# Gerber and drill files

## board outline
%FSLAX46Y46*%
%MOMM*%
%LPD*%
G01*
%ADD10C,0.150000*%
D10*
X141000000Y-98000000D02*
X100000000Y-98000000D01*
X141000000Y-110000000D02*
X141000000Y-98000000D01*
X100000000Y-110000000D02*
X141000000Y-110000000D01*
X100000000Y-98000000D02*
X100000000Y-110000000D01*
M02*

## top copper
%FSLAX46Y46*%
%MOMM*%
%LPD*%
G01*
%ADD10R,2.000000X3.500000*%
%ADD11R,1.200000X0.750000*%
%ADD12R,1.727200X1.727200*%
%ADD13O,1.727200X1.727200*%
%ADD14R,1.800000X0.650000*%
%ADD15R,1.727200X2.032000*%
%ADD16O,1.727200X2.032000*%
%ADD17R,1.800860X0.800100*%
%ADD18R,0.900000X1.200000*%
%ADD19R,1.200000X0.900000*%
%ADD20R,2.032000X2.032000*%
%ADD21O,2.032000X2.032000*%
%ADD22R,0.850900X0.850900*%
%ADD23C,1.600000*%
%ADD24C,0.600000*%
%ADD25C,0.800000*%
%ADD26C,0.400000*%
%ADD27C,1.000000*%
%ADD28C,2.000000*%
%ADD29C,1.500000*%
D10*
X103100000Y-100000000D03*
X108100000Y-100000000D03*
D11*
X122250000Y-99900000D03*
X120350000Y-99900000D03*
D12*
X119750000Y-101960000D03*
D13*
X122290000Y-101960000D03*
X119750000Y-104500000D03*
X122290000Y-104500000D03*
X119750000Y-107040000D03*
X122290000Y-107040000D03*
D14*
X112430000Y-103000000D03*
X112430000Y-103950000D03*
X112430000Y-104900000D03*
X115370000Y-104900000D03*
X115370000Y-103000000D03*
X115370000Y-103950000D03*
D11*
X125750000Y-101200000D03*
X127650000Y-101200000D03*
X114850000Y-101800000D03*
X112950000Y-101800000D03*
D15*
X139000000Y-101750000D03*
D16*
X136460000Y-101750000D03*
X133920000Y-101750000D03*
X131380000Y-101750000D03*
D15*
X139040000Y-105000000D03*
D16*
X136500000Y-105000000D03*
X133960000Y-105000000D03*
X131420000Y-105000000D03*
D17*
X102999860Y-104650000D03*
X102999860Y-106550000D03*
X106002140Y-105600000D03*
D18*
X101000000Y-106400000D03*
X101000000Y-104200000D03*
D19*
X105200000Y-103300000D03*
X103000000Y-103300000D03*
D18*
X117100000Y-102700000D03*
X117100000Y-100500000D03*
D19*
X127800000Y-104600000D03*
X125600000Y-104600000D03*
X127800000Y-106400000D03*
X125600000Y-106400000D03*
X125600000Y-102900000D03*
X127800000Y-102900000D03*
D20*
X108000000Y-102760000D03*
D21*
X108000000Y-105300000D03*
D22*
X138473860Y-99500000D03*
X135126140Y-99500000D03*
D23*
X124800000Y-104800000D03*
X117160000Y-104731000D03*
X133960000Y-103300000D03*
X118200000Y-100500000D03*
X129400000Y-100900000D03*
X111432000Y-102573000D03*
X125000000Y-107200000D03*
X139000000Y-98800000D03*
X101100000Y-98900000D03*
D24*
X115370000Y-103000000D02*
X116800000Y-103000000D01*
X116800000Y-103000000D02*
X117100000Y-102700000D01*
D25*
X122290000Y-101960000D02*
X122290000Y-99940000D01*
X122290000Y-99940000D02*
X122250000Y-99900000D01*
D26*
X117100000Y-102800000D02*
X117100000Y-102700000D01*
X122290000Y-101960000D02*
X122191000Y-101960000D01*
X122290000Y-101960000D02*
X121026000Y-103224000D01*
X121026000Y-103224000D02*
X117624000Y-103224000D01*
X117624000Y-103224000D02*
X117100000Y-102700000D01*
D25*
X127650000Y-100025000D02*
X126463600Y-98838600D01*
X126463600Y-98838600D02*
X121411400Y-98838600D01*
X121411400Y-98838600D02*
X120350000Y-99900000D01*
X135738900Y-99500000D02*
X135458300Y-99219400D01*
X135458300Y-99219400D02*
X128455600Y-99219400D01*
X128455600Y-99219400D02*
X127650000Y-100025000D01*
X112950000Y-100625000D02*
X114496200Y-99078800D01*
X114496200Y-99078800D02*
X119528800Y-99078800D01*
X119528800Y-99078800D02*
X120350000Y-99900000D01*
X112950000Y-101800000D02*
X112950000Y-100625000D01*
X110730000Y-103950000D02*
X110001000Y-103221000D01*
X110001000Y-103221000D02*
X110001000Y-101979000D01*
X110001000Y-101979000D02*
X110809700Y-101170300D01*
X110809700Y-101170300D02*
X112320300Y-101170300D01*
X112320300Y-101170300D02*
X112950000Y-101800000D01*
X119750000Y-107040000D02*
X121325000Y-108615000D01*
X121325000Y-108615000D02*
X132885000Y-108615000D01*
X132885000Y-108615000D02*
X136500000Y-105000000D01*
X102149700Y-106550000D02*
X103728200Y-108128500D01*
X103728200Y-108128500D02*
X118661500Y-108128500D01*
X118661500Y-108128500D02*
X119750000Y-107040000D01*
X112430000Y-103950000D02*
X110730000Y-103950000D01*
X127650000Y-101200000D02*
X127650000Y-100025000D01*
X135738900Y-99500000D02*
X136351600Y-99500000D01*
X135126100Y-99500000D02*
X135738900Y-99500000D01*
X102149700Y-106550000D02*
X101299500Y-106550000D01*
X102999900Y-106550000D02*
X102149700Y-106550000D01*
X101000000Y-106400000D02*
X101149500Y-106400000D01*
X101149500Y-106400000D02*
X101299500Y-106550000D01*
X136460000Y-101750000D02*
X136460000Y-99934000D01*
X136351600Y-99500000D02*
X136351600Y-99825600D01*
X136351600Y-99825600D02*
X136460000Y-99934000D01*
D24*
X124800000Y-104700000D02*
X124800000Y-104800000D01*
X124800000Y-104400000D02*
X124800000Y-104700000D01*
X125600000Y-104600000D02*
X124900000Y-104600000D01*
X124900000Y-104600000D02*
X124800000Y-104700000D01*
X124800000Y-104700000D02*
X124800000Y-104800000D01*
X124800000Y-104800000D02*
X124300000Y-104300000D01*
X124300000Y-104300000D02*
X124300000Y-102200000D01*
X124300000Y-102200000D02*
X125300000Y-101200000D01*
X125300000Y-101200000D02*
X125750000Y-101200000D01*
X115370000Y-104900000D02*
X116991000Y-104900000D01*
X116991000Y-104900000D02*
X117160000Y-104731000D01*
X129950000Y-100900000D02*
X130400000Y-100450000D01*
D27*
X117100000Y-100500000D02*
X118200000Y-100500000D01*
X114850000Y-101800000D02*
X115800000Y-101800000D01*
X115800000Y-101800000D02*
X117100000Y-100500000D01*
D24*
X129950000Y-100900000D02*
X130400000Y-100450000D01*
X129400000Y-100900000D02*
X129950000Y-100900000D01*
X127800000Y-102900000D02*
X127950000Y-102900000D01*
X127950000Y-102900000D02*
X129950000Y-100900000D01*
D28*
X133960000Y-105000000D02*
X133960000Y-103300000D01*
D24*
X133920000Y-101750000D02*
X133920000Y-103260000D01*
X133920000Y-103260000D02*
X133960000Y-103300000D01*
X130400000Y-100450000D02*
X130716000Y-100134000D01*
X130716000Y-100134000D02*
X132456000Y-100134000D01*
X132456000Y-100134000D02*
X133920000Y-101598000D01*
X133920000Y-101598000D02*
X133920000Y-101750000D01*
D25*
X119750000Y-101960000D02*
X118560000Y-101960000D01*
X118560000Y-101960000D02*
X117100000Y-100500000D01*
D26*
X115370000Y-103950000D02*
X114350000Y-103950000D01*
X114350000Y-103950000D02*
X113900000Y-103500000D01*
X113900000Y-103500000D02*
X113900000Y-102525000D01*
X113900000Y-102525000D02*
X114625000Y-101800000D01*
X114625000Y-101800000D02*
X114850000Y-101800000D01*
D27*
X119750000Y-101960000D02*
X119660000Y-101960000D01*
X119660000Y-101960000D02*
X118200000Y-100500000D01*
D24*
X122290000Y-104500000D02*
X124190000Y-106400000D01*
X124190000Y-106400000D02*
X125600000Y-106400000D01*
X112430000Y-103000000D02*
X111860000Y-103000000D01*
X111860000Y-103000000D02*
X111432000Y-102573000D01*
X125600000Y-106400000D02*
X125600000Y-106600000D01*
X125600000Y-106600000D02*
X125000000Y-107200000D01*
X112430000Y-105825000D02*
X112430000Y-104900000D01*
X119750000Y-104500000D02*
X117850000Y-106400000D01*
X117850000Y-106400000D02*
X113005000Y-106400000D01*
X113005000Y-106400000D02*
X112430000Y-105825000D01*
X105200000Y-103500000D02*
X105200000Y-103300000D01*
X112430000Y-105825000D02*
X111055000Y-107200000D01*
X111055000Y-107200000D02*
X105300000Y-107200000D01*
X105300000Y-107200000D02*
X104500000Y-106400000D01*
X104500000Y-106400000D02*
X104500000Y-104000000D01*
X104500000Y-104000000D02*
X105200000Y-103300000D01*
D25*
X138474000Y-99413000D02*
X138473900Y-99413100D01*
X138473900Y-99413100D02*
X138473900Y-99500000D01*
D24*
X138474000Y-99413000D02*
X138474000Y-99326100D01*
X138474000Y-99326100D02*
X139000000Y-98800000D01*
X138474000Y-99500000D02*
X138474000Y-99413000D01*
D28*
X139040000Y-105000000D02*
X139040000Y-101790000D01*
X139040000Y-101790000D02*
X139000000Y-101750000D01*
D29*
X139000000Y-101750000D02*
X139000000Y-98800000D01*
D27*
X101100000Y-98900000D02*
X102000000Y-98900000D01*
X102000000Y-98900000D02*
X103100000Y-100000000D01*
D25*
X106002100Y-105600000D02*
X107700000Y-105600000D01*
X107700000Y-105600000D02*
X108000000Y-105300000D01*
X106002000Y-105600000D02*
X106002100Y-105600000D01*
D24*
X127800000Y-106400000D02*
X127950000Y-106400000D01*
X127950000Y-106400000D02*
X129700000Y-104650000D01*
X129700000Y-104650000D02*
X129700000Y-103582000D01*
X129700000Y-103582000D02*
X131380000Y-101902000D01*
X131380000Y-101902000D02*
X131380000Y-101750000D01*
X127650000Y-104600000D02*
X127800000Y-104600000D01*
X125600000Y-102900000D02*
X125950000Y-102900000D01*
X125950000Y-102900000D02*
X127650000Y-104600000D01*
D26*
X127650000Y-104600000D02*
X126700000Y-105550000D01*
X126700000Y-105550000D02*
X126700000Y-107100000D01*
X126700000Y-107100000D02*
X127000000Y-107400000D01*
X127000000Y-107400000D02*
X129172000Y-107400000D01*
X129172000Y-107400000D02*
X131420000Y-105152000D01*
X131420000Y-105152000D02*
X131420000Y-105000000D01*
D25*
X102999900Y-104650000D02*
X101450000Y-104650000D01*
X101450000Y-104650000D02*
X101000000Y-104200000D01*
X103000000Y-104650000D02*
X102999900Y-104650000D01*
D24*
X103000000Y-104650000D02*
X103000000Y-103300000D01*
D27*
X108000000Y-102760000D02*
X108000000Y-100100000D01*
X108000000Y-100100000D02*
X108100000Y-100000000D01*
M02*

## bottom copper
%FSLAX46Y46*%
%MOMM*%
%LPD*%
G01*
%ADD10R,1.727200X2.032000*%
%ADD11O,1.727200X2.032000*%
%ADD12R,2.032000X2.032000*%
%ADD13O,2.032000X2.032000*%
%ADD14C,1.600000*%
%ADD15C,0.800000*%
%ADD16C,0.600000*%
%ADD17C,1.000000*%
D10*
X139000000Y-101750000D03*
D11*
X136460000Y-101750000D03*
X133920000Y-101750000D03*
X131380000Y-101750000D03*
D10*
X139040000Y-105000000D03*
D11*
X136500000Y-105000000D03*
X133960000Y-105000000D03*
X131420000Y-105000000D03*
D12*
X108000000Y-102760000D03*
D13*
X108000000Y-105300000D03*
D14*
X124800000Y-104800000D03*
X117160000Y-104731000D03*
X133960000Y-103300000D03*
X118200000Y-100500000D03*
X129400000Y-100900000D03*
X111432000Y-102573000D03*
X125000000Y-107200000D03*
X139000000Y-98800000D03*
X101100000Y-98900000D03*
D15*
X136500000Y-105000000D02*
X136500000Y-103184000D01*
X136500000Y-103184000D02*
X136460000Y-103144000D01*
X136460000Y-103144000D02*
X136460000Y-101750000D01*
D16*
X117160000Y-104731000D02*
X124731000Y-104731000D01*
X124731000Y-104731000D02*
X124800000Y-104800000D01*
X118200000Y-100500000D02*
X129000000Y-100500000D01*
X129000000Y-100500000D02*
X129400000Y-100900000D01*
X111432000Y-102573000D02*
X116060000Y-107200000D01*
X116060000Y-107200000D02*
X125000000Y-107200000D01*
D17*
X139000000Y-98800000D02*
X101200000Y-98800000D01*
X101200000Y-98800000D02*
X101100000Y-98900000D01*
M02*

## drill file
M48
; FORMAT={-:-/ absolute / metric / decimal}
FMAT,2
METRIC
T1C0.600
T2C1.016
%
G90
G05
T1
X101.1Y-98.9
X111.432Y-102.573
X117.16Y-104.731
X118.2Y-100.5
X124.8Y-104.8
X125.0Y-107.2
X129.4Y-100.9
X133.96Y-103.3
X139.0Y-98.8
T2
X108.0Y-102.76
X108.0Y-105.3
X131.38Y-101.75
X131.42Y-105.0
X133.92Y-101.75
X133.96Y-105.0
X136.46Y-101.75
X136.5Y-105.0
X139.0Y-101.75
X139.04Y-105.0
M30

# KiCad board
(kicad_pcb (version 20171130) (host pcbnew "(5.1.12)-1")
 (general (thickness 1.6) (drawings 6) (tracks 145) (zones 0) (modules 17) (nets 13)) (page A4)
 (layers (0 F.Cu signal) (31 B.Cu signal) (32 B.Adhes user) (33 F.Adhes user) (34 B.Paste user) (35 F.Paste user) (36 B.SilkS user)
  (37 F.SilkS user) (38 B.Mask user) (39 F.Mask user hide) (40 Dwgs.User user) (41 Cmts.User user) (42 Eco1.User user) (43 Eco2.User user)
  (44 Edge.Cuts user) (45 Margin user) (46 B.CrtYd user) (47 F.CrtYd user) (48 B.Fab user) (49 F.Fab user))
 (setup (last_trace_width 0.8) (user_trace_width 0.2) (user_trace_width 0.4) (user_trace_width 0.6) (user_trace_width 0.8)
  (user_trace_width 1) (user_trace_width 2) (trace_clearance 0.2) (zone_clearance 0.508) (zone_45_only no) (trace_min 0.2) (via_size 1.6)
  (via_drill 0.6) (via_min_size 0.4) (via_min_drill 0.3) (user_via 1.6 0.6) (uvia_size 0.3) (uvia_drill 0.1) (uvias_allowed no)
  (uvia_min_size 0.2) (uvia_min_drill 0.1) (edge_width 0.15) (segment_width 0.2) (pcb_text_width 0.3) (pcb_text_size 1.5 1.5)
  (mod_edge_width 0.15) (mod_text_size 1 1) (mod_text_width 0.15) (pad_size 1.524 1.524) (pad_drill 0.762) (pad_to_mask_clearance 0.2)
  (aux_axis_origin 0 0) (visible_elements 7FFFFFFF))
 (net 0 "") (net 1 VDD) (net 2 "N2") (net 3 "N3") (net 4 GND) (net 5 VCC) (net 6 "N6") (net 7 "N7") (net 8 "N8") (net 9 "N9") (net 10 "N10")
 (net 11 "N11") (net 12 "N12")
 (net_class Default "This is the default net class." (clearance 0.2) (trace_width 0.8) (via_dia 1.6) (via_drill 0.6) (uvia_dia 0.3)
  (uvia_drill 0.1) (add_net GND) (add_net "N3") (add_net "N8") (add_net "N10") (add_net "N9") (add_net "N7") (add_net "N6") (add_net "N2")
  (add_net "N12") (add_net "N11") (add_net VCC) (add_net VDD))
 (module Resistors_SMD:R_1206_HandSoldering (layer F.Cu) (at 105.6 100)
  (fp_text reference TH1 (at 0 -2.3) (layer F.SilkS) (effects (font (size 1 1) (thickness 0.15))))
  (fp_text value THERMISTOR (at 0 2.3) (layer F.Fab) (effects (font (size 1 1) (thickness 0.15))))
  (pad 1 smd rect (at -2.5 0) (size 2 3.5) (layers F.Cu F.Paste F.Mask) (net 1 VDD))
  (pad 2 smd rect (at 2.5 0) (size 2 3.5) (layers F.Cu F.Paste F.Mask) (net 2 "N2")))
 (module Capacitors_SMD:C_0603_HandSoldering (layer F.Cu) (at 121.3 99.9 180)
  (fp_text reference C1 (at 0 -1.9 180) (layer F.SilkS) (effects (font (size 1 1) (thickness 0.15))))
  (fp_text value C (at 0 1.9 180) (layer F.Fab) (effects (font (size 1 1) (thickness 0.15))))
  (pad 1 smd rect (at -0.95 0 180) (size 1.2 0.75) (layers F.Cu F.Paste F.Mask) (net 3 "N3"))
  (pad 2 smd rect (at 0.95 0 180) (size 1.2 0.75) (layers F.Cu F.Paste F.Mask) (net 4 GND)))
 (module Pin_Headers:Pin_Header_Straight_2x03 (layer F.Cu) (at 119.75 101.96)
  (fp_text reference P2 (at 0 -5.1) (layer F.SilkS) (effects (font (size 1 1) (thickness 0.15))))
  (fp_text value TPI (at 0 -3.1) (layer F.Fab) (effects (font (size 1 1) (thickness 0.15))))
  (pad 1 smd rect (at 0 0) (size 1.7272 1.7272) (layers F.Cu F.Paste F.Mask) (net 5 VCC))
  (pad 2 smd oval (at 2.54 0) (size 1.7272 1.7272) (layers F.Cu F.Paste F.Mask) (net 3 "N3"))
  (pad 3 smd oval (at 0 2.54) (size 1.7272 1.7272) (layers F.Cu F.Paste F.Mask) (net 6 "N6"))
  (pad 4 smd oval (at 2.54 2.54) (size 1.7272 1.7272) (layers F.Cu F.Paste F.Mask) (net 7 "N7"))
  (pad 5 smd oval (at 0 5.08) (size 1.7272 1.7272) (layers F.Cu F.Paste F.Mask) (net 4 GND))
  (pad 6 smd oval (at 2.54 5.08) (size 1.7272 1.7272) (layers F.Cu F.Paste F.Mask)))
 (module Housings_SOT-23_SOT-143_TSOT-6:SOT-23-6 (layer F.Cu) (at 113.9 103.95)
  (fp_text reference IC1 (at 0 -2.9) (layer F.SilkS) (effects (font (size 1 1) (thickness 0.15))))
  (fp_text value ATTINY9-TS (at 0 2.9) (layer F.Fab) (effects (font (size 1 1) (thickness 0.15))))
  (pad 1 smd rect (at -1.47 -0.95) (size 1.8 0.65) (layers F.Cu F.Paste F.Mask) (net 7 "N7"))
  (pad 2 smd rect (at -1.47 0) (size 1.8 0.65) (layers F.Cu F.Paste F.Mask) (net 4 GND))
  (pad 3 smd rect (at -1.47 0.95) (size 1.8 0.65) (layers F.Cu F.Paste F.Mask) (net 6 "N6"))
  (pad 4 smd rect (at 1.47 0.95) (size 1.8 0.65) (layers F.Cu F.Paste F.Mask) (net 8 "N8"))
  (pad 6 smd rect (at 1.47 -0.95) (size 1.8 0.65) (layers F.Cu F.Paste F.Mask) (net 3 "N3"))
  (pad 5 smd rect (at 1.47 0) (size 1.8 0.65) (layers F.Cu F.Paste F.Mask) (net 5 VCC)))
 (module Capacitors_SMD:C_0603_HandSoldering (layer F.Cu) (at 126.7 101.2)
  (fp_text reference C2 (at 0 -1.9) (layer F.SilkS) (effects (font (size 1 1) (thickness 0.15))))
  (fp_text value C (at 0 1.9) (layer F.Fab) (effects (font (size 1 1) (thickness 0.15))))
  (pad 1 smd rect (at -0.95 0) (size 1.2 0.75) (layers F.Cu F.Paste F.Mask) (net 8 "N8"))
  (pad 2 smd rect (at 0.95 0) (size 1.2 0.75) (layers F.Cu F.Paste F.Mask) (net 4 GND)))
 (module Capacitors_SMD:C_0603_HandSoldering (layer F.Cu) (at 113.9 101.8 180)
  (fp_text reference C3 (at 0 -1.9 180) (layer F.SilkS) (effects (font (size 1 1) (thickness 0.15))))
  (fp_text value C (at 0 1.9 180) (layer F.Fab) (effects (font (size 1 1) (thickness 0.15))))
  (pad 1 smd rect (at -0.95 0 180) (size 1.2 0.75) (layers F.Cu F.Paste F.Mask) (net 5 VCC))
  (pad 2 smd rect (at 0.95 0 180) (size 1.2 0.75) (layers F.Cu F.Paste F.Mask) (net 4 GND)))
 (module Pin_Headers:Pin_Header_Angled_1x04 (layer B.Cu) (at 139 101.75 90)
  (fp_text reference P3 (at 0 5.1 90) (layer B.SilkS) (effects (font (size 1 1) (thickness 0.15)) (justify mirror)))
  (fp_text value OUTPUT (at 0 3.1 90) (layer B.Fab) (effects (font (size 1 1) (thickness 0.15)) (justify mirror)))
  (pad 1 thru_hole rect (at 0 0 90) (size 2.032 1.7272) (drill 1.016) (layers *.Cu *.Mask B.SilkS) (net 1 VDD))
  (pad 2 thru_hole oval (at 0 -2.54 90) (size 2.032 1.7272) (drill 1.016) (layers *.Cu *.Mask B.SilkS) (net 4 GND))
  (pad 3 thru_hole oval (at 0 -5.08 90) (size 2.032 1.7272) (drill 1.016) (layers *.Cu *.Mask B.SilkS) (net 5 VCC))
  (pad 4 thru_hole oval (at 0 -7.62 90) (size 2.032 1.7272) (drill 1.016) (layers *.Cu *.Mask B.SilkS) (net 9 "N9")))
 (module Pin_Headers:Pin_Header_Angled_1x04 (layer F.Cu) (at 139.04 105 270)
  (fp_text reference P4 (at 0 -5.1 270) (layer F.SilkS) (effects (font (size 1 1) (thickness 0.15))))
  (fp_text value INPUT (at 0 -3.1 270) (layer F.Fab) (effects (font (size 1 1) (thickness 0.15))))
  (pad 1 thru_hole rect (at 0 0 270) (size 2.032 1.7272) (drill 1.016) (layers *.Cu *.Mask F.SilkS) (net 1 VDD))
  (pad 2 thru_hole oval (at 0 2.54 270) (size 2.032 1.7272) (drill 1.016) (layers *.Cu *.Mask F.SilkS) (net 4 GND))
  (pad 3 thru_hole oval (at 0 5.08 270) (size 2.032 1.7272) (drill 1.016) (layers *.Cu *.Mask F.SilkS) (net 5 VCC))
  (pad 4 thru_hole oval (at 0 7.62 270) (size 2.032 1.7272) (drill 1.016) (layers *.Cu *.Mask F.SilkS) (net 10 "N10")))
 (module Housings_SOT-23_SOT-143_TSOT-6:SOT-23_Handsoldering (layer F.Cu) (at 104.501 105.6 270)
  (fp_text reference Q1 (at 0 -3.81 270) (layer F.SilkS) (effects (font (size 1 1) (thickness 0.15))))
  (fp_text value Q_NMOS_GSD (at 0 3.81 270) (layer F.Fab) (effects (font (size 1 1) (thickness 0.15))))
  (pad 1 smd rect (at -0.95 1.50114 270) (size 0.8001 1.80086) (layers F.Cu F.Paste F.Mask) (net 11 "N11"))
  (pad 2 smd rect (at 0.95 1.50114 270) (size 0.8001 1.80086) (layers F.Cu F.Paste F.Mask) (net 4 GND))
  (pad 3 smd rect (at 0 -1.50114 270) (size 0.8001 1.80086) (layers F.Cu F.Paste F.Mask) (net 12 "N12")))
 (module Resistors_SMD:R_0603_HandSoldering (layer F.Cu) (at 101 105.3 90)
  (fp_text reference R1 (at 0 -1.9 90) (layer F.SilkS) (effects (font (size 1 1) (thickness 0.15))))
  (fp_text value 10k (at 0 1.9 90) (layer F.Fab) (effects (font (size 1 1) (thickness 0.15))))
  (pad 1 smd rect (at -1.1 0 90) (size 1.2 0.9) (layers F.Cu F.Paste F.Mask) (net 4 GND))
  (pad 2 smd rect (at 1.1 0 90) (size 1.2 0.9) (layers F.Cu F.Paste F.Mask) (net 11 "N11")))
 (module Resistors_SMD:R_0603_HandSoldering (layer F.Cu) (at 104.1 103.3 180)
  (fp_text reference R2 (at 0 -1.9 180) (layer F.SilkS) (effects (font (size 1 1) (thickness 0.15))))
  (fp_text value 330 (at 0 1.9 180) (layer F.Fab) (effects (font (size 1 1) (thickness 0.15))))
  (pad 1 smd rect (at -1.1 0 180) (size 1.2 0.9) (layers F.Cu F.Paste F.Mask) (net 6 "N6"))
  (pad 2 smd rect (at 1.1 0 180) (size 1.2 0.9) (layers F.Cu F.Paste F.Mask) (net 11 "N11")))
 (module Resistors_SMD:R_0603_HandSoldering (layer F.Cu) (at 117.1 101.6 90)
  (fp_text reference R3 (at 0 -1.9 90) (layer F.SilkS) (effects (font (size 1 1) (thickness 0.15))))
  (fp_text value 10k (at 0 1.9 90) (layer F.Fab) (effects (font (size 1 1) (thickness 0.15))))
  (pad 1 smd rect (at -1.1 0 90) (size 1.2 0.9) (layers F.Cu F.Paste F.Mask) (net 3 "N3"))
  (pad 2 smd rect (at 1.1 0 90) (size 1.2 0.9) (layers F.Cu F.Paste F.Mask) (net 5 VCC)))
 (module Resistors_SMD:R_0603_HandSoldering (layer F.Cu) (at 126.7 104.6 180)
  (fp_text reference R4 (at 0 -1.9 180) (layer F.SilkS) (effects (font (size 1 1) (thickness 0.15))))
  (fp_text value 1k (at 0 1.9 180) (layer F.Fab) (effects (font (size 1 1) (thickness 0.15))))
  (pad 1 smd rect (at -1.1 0 180) (size 1.2 0.9) (layers F.Cu F.Paste F.Mask) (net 10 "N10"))
  (pad 2 smd rect (at 1.1 0 180) (size 1.2 0.9) (layers F.Cu F.Paste F.Mask) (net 8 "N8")))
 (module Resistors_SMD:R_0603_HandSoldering (layer F.Cu) (at 126.7 106.4 180)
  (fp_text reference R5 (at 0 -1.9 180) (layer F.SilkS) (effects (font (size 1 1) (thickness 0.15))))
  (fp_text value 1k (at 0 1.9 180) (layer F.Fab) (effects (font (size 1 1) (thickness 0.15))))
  (pad 1 smd rect (at -1.1 0 180) (size 1.2 0.9) (layers F.Cu F.Paste F.Mask) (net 9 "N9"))
  (pad 2 smd rect (at 1.1 0 180) (size 1.2 0.9) (layers F.Cu F.Paste F.Mask) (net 7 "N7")))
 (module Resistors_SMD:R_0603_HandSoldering (layer F.Cu) (at 126.7 102.9)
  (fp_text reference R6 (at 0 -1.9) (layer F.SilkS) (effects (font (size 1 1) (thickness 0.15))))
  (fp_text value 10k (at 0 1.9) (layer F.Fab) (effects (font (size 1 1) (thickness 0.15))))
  (pad 1 smd rect (at -1.1 0) (size 1.2 0.9) (layers F.Cu F.Paste F.Mask) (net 10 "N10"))
  (pad 2 smd rect (at 1.1 0) (size 1.2 0.9) (layers F.Cu F.Paste F.Mask) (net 5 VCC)))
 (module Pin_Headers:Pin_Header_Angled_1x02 (layer B.Cu) (at 108 102.76 180)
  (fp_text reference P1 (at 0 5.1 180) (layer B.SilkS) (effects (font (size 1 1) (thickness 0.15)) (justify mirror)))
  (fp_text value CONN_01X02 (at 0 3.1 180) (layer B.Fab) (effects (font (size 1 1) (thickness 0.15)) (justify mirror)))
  (pad 1 thru_hole rect (at 0 0 180) (size 2.032 2.032) (drill 1.016) (layers *.Cu *.Mask B.SilkS) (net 2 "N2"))
  (pad 2 thru_hole oval (at 0 -2.54 180) (size 2.032 2.032) (drill 1.016) (layers *.Cu *.Mask B.SilkS) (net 12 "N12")))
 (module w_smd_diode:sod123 (layer F.Cu) (at 136.8 99.5)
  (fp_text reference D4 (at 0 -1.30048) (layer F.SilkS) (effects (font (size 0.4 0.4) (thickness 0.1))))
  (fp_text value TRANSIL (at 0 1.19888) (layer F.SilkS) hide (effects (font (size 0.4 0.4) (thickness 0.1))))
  (pad 2 smd rect (at 1.67386 0) (size 0.8509 0.8509) (layers F.Cu F.Paste F.Mask) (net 1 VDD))
  (pad 1 smd rect (at -1.67386 0) (size 0.8509 0.8509) (layers F.Cu F.Paste F.Mask) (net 4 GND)))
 (gr_line (start 141 98) (end 100 98) (layer Edge.Cuts) (width 0.15))
 (gr_line (start 141 110) (end 141 98) (layer Edge.Cuts) (width 0.15))
 (gr_line (start 100 110) (end 141 110) (layer Edge.Cuts) (width 0.15))
 (gr_line (start 100 98) (end 100 110) (layer Edge.Cuts) (width 0.15))
 (segment (start 115.37 103) (end 116.8 103) (width 0.6) (layer F.Cu) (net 3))
 (segment (start 116.8 103) (end 117.1 102.7) (width 0.6) (layer F.Cu) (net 3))
 (segment (start 122.29 101.96) (end 122.29 99.94) (width 0.8) (layer F.Cu) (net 3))
 (segment (start 122.29 99.94) (end 122.25 99.9) (width 0.8) (layer F.Cu) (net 3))
 (segment (start 117.1 102.8) (end 117.1 102.7) (width 0.4) (layer F.Cu) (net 3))
 (segment (start 122.29 101.96) (end 122.191 101.96) (width 0.4) (layer F.Cu) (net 3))
 (segment (start 122.29 101.96) (end 121.026 103.224) (width 0.4) (layer F.Cu) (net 3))
 (segment (start 121.026 103.224) (end 117.624 103.224) (width 0.4) (layer F.Cu) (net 3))
 (segment (start 117.624 103.224) (end 117.1 102.7) (width 0.4) (layer F.Cu) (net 3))
 (segment (start 127.65 100.025) (end 126.4636 98.8386) (width 0.8) (layer F.Cu) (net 4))
 (segment (start 126.4636 98.8386) (end 121.4114 98.8386) (width 0.8) (layer F.Cu) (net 4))
 (segment (start 121.4114 98.8386) (end 120.35 99.9) (width 0.8) (layer F.Cu) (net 4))
 (segment (start 135.7389 99.5) (end 135.4583 99.2194) (width 0.8) (layer F.Cu) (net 4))
 (segment (start 135.4583 99.2194) (end 128.4556 99.2194) (width 0.8) (layer F.Cu) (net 4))
 (segment (start 128.4556 99.2194) (end 127.65 100.025) (width 0.8) (layer F.Cu) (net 4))
 (segment (start 112.95 100.625) (end 114.4962 99.0788) (width 0.8) (layer F.Cu) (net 4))
 (segment (start 114.4962 99.0788) (end 119.5288 99.0788) (width 0.8) (layer F.Cu) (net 4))
 (segment (start 119.5288 99.0788) (end 120.35 99.9) (width 0.8) (layer F.Cu) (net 4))
 (segment (start 112.95 101.8) (end 112.95 100.625) (width 0.8) (layer F.Cu) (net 4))
 (segment (start 110.73 103.95) (end 110.001 103.221) (width 0.8) (layer F.Cu) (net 4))
 (segment (start 110.001 103.221) (end 110.001 101.979) (width 0.8) (layer F.Cu) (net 4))
 (segment (start 110.001 101.979) (end 110.8097 101.1703) (width 0.8) (layer F.Cu) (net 4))
 (segment (start 110.8097 101.1703) (end 112.3203 101.1703) (width 0.8) (layer F.Cu) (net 4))
 (segment (start 112.3203 101.1703) (end 112.95 101.8) (width 0.8) (layer F.Cu) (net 4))
 (segment (start 119.75 107.04) (end 121.325 108.615) (width 0.8) (layer F.Cu) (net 4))
 (segment (start 121.325 108.615) (end 132.885 108.615) (width 0.8) (layer F.Cu) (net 4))
 (segment (start 132.885 108.615) (end 136.5 105) (width 0.8) (layer F.Cu) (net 4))
 (segment (start 102.1497 106.55) (end 103.7282 108.1285) (width 0.8) (layer F.Cu) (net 4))
 (segment (start 103.7282 108.1285) (end 118.6615 108.1285) (width 0.8) (layer F.Cu) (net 4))
 (segment (start 118.6615 108.1285) (end 119.75 107.04) (width 0.8) (layer F.Cu) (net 4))
 (segment (start 112.43 103.95) (end 110.73 103.95) (width 0.8) (layer F.Cu) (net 4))
 (segment (start 127.65 101.2) (end 127.65 100.025) (width 0.8) (layer F.Cu) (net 4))
 (segment (start 135.7389 99.5) (end 136.3516 99.5) (width 0.8) (layer F.Cu) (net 4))
 (segment (start 135.1261 99.5) (end 135.7389 99.5) (width 0.8) (layer F.Cu) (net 4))
 (segment (start 136.5 105) (end 136.5 103.184) (width 0.8) (layer B.Cu) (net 4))
 (segment (start 136.5 103.184) (end 136.46 103.144) (width 0.8) (layer B.Cu) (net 4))
 (segment (start 136.46 103.144) (end 136.46 101.75) (width 0.8) (layer B.Cu) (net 4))
 (segment (start 102.1497 106.55) (end 101.2995 106.55) (width 0.8) (layer F.Cu) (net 4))
 (segment (start 102.9999 106.55) (end 102.1497 106.55) (width 0.8) (layer F.Cu) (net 4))
 (segment (start 101 106.4) (end 101.1495 106.4) (width 0.8) (layer F.Cu) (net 4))
 (segment (start 101.1495 106.4) (end 101.2995 106.55) (width 0.8) (layer F.Cu) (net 4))
 (segment (start 136.46 101.75) (end 136.46 99.934) (width 0.8) (layer F.Cu) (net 4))
 (segment (start 136.3516 99.5) (end 136.3516 99.8256) (width 0.8) (layer F.Cu) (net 4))
 (segment (start 136.3516 99.8256) (end 136.46 99.934) (width 0.8) (layer F.Cu) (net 4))
 (segment (start 124.8 104.7) (end 124.8 104.8) (width 0.6) (layer F.Cu) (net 8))
 (segment (start 124.8 104.4) (end 124.8 104.7) (width 0.6) (layer F.Cu) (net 8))
 (segment (start 125.6 104.6) (end 124.9 104.6) (width 0.6) (layer F.Cu) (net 8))
 (segment (start 124.9 104.6) (end 124.8 104.7) (width 0.6) (layer F.Cu) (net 8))
 (segment (start 124.8 104.7) (end 124.8 104.8) (width 0.6) (layer F.Cu) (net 8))
 (segment (start 124.8 104.8) (end 124.3 104.3) (width 0.6) (layer F.Cu) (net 8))
 (segment (start 124.3 104.3) (end 124.3 102.2) (width 0.6) (layer F.Cu) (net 8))
 (segment (start 124.3 102.2) (end 125.3 101.2) (width 0.6) (layer F.Cu) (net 8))
 (segment (start 125.3 101.2) (end 125.75 101.2) (width 0.6) (layer F.Cu) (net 8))
 (segment (start 115.37 104.9) (end 116.991 104.9) (width 0.6) (layer F.Cu) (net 8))
 (segment (start 116.991 104.9) (end 117.16 104.731) (width 0.6) (layer F.Cu) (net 8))
 (segment (start 117.16 104.731) (end 124.731 104.731) (width 0.6) (layer B.Cu) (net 8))
 (segment (start 124.731 104.731) (end 124.8 104.8) (width 0.6) (layer B.Cu) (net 8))
 (via (at 124.8 104.8) (size 1.6) (layers F.Cu B.Cu) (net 8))
 (via (at 117.16 104.731) (size 1.6) (layers F.Cu B.Cu) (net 8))
 (segment (start 129.95 100.9) (end 130.4 100.45) (width 0.6) (layer F.Cu) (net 5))
 (segment (start 117.1 100.5) (end 118.2 100.5) (width 1) (layer F.Cu) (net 5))
 (segment (start 114.85 101.8) (end 115.8 101.8) (width 1) (layer F.Cu) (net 5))
 (segment (start 115.8 101.8) (end 117.1 100.5) (width 1) (layer F.Cu) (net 5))
 (segment (start 129.95 100.9) (end 130.4 100.45) (width 0.6) (layer F.Cu) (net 5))
 (segment (start 129.4 100.9) (end 129.95 100.9) (width 0.6) (layer F.Cu) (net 5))
 (segment (start 127.8 102.9) (end 127.95 102.9) (width 0.6) (layer F.Cu) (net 5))
 (segment (start 127.95 102.9) (end 129.95 100.9) (width 0.6) (layer F.Cu) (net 5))
 (segment (start 133.96 105) (end 133.96 103.3) (width 2) (layer F.Cu) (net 5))
 (segment (start 133.92 101.75) (end 133.92 103.26) (width 0.6) (layer F.Cu) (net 5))
 (segment (start 133.92 103.26) (end 133.96 103.3) (width 0.6) (layer F.Cu) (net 5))
 (segment (start 130.4 100.45) (end 130.716 100.134) (width 0.6) (layer F.Cu) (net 5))
 (segment (start 130.716 100.134) (end 132.456 100.134) (width 0.6) (layer F.Cu) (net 5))
 (segment (start 132.456 100.134) (end 133.92 101.598) (width 0.6) (layer F.Cu) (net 5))
 (segment (start 133.92 101.598) (end 133.92 101.75) (width 0.6) (layer F.Cu) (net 5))
 (segment (start 119.75 101.96) (end 118.56 101.96) (width 0.8) (layer F.Cu) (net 5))
 (segment (start 118.56 101.96) (end 117.1 100.5) (width 0.8) (layer F.Cu) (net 5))
 (segment (start 115.37 103.95) (end 114.35 103.95) (width 0.4) (layer F.Cu) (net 5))
 (segment (start 114.35 103.95) (end 113.9 103.5) (width 0.4) (layer F.Cu) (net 5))
 (segment (start 113.9 103.5) (end 113.9 102.525) (width 0.4) (layer F.Cu) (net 5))
 (segment (start 113.9 102.525) (end 114.625 101.8) (width 0.4) (layer F.Cu) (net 5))
 (segment (start 114.625 101.8) (end 114.85 101.8) (width 0.4) (layer F.Cu) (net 5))
 (segment (start 118.2 100.5) (end 129 100.5) (width 0.6) (layer B.Cu) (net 5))
 (segment (start 129 100.5) (end 129.4 100.9) (width 0.6) (layer B.Cu) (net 5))
 (segment (start 119.75 101.96) (end 119.66 101.96) (width 1) (layer F.Cu) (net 5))
 (segment (start 119.66 101.96) (end 118.2 100.5) (width 1) (layer F.Cu) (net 5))
 (via (at 133.96 103.3) (size 1.6) (layers F.Cu B.Cu) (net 5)) (via (at 118.2 100.5) (size 1.6) (layers F.Cu B.Cu) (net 5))
 (via (at 129.4 100.9) (size 1.6) (layers F.Cu B.Cu) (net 5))
 (segment (start 122.29 104.5) (end 124.19 106.4) (width 0.6) (layer F.Cu) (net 7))
 (segment (start 124.19 106.4) (end 125.6 106.4) (width 0.6) (layer F.Cu) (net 7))
 (segment (start 112.43 103) (end 111.86 103) (width 0.6) (layer F.Cu) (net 7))
 (segment (start 111.86 103) (end 111.432 102.573) (width 0.6) (layer F.Cu) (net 7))
 (segment (start 125.6 106.4) (end 125.6 106.6) (width 0.6) (layer F.Cu) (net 7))
 (segment (start 125.6 106.6) (end 125 107.2) (width 0.6) (layer F.Cu) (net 7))
 (segment (start 111.432 102.573) (end 116.06 107.2) (width 0.6) (layer B.Cu) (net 7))
 (segment (start 116.06 107.2) (end 125 107.2) (width 0.6) (layer B.Cu) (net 7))
 (via (at 111.432 102.573) (size 1.6) (layers F.Cu B.Cu) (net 7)) (via (at 125 107.2) (size 1.6) (layers F.Cu B.Cu) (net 7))
 (segment (start 112.43 105.825) (end 112.43 104.9) (width 0.6) (layer F.Cu) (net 6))
 (segment (start 119.75 104.5) (end 117.85 106.4) (width 0.6) (layer F.Cu) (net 6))
 (segment (start 117.85 106.4) (end 113.005 106.4) (width 0.6) (layer F.Cu) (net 6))
 (segment (start 113.005 106.4) (end 112.43 105.825) (width 0.6) (layer F.Cu) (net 6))
 (segment (start 105.2 103.5) (end 105.2 103.3) (width 0.6) (layer F.Cu) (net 6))
 (segment (start 112.43 105.825) (end 111.055 107.2) (width 0.6) (layer F.Cu) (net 6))
 (segment (start 111.055 107.2) (end 105.3 107.2) (width 0.6) (layer F.Cu) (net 6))
 (segment (start 105.3 107.2) (end 104.5 106.4) (width 0.6) (layer F.Cu) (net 6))
 (segment (start 104.5 106.4) (end 104.5 104) (width 0.6) (layer F.Cu) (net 6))
 (segment (start 104.5 104) (end 105.2 103.3) (width 0.6) (layer F.Cu) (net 6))
 (segment (start 138.474 99.413) (end 138.4739 99.4131) (width 0.8) (layer F.Cu) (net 1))
 (segment (start 138.4739 99.4131) (end 138.4739 99.5) (width 0.8) (layer F.Cu) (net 1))
 (segment (start 138.474 99.413) (end 138.474 99.3261) (width 0.6) (layer F.Cu) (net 1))
 (segment (start 138.474 99.3261) (end 139 98.8) (width 0.6) (layer F.Cu) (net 1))
 (segment (start 138.474 99.5) (end 138.474 99.413) (width 0.6) (layer F.Cu) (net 1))
 (segment (start 139.04 105) (end 139.04 101.79) (width 2) (layer F.Cu) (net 1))
 (segment (start 139.04 101.79) (end 139 101.75) (width 2) (layer F.Cu) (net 1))
 (segment (start 139 101.75) (end 139 98.8) (width 1.5) (layer F.Cu) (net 1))
 (segment (start 139 98.8) (end 101.2 98.8) (width 1) (layer B.Cu) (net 1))
 (segment (start 101.2 98.8) (end 101.1 98.9) (width 1) (layer B.Cu) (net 1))
 (segment (start 101.1 98.9) (end 102 98.9) (width 1) (layer F.Cu) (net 1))
 (segment (start 102 98.9) (end 103.1 100) (width 1) (layer F.Cu) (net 1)) (via (at 139 98.8) (size 1.6) (layers F.Cu B.Cu) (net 1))
 (via (at 101.1 98.9) (size 1.6) (layers F.Cu B.Cu) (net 1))
 (segment (start 106.0021 105.6) (end 107.7 105.6) (width 0.8) (layer F.Cu) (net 12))
 (segment (start 107.7 105.6) (end 108 105.3) (width 0.8) (layer F.Cu) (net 12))
 (segment (start 106.002 105.6) (end 106.0021 105.6) (width 0.8) (layer F.Cu) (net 12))
 (segment (start 127.8 106.4) (end 127.95 106.4) (width 0.6) (layer F.Cu) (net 9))
 (segment (start 127.95 106.4) (end 129.7 104.65) (width 0.6) (layer F.Cu) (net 9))
 (segment (start 129.7 104.65) (end 129.7 103.582) (width 0.6) (layer F.Cu) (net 9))
 (segment (start 129.7 103.582) (end 131.38 101.902) (width 0.6) (layer F.Cu) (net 9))
 (segment (start 131.38 101.902) (end 131.38 101.75) (width 0.6) (layer F.Cu) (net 9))
 (segment (start 127.65 104.6) (end 127.8 104.6) (width 0.6) (layer F.Cu) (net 10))
 (segment (start 125.6 102.9) (end 125.95 102.9) (width 0.6) (layer F.Cu) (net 10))
 (segment (start 125.95 102.9) (end 127.65 104.6) (width 0.6) (layer F.Cu) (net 10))
 (segment (start 127.65 104.6) (end 126.7 105.55) (width 0.4) (layer F.Cu) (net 10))
 (segment (start 126.7 105.55) (end 126.7 107.1) (width 0.4) (layer F.Cu) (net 10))
 (segment (start 126.7 107.1) (end 127 107.4) (width 0.4) (layer F.Cu) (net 10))
 (segment (start 127 107.4) (end 129.172 107.4) (width 0.4) (layer F.Cu) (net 10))
 (segment (start 129.172 107.4) (end 131.42 105.152) (width 0.4) (layer F.Cu) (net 10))
 (segment (start 131.42 105.152) (end 131.42 105) (width 0.4) (layer F.Cu) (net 10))
 (segment (start 102.9999 104.65) (end 101.45 104.65) (width 0.8) (layer F.Cu) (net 11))
 (segment (start 101.45 104.65) (end 101 104.2) (width 0.8) (layer F.Cu) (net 11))
 (segment (start 103 104.65) (end 102.9999 104.65) (width 0.8) (layer F.Cu) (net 11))
 (segment (start 103 104.65) (end 103 103.3) (width 0.6) (layer F.Cu) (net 11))
 (segment (start 108 102.76) (end 108 100.1) (width 1) (layer F.Cu) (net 2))
 (segment (start 108 100.1) (end 108.1 100) (width 1) (layer F.Cu) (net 2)))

